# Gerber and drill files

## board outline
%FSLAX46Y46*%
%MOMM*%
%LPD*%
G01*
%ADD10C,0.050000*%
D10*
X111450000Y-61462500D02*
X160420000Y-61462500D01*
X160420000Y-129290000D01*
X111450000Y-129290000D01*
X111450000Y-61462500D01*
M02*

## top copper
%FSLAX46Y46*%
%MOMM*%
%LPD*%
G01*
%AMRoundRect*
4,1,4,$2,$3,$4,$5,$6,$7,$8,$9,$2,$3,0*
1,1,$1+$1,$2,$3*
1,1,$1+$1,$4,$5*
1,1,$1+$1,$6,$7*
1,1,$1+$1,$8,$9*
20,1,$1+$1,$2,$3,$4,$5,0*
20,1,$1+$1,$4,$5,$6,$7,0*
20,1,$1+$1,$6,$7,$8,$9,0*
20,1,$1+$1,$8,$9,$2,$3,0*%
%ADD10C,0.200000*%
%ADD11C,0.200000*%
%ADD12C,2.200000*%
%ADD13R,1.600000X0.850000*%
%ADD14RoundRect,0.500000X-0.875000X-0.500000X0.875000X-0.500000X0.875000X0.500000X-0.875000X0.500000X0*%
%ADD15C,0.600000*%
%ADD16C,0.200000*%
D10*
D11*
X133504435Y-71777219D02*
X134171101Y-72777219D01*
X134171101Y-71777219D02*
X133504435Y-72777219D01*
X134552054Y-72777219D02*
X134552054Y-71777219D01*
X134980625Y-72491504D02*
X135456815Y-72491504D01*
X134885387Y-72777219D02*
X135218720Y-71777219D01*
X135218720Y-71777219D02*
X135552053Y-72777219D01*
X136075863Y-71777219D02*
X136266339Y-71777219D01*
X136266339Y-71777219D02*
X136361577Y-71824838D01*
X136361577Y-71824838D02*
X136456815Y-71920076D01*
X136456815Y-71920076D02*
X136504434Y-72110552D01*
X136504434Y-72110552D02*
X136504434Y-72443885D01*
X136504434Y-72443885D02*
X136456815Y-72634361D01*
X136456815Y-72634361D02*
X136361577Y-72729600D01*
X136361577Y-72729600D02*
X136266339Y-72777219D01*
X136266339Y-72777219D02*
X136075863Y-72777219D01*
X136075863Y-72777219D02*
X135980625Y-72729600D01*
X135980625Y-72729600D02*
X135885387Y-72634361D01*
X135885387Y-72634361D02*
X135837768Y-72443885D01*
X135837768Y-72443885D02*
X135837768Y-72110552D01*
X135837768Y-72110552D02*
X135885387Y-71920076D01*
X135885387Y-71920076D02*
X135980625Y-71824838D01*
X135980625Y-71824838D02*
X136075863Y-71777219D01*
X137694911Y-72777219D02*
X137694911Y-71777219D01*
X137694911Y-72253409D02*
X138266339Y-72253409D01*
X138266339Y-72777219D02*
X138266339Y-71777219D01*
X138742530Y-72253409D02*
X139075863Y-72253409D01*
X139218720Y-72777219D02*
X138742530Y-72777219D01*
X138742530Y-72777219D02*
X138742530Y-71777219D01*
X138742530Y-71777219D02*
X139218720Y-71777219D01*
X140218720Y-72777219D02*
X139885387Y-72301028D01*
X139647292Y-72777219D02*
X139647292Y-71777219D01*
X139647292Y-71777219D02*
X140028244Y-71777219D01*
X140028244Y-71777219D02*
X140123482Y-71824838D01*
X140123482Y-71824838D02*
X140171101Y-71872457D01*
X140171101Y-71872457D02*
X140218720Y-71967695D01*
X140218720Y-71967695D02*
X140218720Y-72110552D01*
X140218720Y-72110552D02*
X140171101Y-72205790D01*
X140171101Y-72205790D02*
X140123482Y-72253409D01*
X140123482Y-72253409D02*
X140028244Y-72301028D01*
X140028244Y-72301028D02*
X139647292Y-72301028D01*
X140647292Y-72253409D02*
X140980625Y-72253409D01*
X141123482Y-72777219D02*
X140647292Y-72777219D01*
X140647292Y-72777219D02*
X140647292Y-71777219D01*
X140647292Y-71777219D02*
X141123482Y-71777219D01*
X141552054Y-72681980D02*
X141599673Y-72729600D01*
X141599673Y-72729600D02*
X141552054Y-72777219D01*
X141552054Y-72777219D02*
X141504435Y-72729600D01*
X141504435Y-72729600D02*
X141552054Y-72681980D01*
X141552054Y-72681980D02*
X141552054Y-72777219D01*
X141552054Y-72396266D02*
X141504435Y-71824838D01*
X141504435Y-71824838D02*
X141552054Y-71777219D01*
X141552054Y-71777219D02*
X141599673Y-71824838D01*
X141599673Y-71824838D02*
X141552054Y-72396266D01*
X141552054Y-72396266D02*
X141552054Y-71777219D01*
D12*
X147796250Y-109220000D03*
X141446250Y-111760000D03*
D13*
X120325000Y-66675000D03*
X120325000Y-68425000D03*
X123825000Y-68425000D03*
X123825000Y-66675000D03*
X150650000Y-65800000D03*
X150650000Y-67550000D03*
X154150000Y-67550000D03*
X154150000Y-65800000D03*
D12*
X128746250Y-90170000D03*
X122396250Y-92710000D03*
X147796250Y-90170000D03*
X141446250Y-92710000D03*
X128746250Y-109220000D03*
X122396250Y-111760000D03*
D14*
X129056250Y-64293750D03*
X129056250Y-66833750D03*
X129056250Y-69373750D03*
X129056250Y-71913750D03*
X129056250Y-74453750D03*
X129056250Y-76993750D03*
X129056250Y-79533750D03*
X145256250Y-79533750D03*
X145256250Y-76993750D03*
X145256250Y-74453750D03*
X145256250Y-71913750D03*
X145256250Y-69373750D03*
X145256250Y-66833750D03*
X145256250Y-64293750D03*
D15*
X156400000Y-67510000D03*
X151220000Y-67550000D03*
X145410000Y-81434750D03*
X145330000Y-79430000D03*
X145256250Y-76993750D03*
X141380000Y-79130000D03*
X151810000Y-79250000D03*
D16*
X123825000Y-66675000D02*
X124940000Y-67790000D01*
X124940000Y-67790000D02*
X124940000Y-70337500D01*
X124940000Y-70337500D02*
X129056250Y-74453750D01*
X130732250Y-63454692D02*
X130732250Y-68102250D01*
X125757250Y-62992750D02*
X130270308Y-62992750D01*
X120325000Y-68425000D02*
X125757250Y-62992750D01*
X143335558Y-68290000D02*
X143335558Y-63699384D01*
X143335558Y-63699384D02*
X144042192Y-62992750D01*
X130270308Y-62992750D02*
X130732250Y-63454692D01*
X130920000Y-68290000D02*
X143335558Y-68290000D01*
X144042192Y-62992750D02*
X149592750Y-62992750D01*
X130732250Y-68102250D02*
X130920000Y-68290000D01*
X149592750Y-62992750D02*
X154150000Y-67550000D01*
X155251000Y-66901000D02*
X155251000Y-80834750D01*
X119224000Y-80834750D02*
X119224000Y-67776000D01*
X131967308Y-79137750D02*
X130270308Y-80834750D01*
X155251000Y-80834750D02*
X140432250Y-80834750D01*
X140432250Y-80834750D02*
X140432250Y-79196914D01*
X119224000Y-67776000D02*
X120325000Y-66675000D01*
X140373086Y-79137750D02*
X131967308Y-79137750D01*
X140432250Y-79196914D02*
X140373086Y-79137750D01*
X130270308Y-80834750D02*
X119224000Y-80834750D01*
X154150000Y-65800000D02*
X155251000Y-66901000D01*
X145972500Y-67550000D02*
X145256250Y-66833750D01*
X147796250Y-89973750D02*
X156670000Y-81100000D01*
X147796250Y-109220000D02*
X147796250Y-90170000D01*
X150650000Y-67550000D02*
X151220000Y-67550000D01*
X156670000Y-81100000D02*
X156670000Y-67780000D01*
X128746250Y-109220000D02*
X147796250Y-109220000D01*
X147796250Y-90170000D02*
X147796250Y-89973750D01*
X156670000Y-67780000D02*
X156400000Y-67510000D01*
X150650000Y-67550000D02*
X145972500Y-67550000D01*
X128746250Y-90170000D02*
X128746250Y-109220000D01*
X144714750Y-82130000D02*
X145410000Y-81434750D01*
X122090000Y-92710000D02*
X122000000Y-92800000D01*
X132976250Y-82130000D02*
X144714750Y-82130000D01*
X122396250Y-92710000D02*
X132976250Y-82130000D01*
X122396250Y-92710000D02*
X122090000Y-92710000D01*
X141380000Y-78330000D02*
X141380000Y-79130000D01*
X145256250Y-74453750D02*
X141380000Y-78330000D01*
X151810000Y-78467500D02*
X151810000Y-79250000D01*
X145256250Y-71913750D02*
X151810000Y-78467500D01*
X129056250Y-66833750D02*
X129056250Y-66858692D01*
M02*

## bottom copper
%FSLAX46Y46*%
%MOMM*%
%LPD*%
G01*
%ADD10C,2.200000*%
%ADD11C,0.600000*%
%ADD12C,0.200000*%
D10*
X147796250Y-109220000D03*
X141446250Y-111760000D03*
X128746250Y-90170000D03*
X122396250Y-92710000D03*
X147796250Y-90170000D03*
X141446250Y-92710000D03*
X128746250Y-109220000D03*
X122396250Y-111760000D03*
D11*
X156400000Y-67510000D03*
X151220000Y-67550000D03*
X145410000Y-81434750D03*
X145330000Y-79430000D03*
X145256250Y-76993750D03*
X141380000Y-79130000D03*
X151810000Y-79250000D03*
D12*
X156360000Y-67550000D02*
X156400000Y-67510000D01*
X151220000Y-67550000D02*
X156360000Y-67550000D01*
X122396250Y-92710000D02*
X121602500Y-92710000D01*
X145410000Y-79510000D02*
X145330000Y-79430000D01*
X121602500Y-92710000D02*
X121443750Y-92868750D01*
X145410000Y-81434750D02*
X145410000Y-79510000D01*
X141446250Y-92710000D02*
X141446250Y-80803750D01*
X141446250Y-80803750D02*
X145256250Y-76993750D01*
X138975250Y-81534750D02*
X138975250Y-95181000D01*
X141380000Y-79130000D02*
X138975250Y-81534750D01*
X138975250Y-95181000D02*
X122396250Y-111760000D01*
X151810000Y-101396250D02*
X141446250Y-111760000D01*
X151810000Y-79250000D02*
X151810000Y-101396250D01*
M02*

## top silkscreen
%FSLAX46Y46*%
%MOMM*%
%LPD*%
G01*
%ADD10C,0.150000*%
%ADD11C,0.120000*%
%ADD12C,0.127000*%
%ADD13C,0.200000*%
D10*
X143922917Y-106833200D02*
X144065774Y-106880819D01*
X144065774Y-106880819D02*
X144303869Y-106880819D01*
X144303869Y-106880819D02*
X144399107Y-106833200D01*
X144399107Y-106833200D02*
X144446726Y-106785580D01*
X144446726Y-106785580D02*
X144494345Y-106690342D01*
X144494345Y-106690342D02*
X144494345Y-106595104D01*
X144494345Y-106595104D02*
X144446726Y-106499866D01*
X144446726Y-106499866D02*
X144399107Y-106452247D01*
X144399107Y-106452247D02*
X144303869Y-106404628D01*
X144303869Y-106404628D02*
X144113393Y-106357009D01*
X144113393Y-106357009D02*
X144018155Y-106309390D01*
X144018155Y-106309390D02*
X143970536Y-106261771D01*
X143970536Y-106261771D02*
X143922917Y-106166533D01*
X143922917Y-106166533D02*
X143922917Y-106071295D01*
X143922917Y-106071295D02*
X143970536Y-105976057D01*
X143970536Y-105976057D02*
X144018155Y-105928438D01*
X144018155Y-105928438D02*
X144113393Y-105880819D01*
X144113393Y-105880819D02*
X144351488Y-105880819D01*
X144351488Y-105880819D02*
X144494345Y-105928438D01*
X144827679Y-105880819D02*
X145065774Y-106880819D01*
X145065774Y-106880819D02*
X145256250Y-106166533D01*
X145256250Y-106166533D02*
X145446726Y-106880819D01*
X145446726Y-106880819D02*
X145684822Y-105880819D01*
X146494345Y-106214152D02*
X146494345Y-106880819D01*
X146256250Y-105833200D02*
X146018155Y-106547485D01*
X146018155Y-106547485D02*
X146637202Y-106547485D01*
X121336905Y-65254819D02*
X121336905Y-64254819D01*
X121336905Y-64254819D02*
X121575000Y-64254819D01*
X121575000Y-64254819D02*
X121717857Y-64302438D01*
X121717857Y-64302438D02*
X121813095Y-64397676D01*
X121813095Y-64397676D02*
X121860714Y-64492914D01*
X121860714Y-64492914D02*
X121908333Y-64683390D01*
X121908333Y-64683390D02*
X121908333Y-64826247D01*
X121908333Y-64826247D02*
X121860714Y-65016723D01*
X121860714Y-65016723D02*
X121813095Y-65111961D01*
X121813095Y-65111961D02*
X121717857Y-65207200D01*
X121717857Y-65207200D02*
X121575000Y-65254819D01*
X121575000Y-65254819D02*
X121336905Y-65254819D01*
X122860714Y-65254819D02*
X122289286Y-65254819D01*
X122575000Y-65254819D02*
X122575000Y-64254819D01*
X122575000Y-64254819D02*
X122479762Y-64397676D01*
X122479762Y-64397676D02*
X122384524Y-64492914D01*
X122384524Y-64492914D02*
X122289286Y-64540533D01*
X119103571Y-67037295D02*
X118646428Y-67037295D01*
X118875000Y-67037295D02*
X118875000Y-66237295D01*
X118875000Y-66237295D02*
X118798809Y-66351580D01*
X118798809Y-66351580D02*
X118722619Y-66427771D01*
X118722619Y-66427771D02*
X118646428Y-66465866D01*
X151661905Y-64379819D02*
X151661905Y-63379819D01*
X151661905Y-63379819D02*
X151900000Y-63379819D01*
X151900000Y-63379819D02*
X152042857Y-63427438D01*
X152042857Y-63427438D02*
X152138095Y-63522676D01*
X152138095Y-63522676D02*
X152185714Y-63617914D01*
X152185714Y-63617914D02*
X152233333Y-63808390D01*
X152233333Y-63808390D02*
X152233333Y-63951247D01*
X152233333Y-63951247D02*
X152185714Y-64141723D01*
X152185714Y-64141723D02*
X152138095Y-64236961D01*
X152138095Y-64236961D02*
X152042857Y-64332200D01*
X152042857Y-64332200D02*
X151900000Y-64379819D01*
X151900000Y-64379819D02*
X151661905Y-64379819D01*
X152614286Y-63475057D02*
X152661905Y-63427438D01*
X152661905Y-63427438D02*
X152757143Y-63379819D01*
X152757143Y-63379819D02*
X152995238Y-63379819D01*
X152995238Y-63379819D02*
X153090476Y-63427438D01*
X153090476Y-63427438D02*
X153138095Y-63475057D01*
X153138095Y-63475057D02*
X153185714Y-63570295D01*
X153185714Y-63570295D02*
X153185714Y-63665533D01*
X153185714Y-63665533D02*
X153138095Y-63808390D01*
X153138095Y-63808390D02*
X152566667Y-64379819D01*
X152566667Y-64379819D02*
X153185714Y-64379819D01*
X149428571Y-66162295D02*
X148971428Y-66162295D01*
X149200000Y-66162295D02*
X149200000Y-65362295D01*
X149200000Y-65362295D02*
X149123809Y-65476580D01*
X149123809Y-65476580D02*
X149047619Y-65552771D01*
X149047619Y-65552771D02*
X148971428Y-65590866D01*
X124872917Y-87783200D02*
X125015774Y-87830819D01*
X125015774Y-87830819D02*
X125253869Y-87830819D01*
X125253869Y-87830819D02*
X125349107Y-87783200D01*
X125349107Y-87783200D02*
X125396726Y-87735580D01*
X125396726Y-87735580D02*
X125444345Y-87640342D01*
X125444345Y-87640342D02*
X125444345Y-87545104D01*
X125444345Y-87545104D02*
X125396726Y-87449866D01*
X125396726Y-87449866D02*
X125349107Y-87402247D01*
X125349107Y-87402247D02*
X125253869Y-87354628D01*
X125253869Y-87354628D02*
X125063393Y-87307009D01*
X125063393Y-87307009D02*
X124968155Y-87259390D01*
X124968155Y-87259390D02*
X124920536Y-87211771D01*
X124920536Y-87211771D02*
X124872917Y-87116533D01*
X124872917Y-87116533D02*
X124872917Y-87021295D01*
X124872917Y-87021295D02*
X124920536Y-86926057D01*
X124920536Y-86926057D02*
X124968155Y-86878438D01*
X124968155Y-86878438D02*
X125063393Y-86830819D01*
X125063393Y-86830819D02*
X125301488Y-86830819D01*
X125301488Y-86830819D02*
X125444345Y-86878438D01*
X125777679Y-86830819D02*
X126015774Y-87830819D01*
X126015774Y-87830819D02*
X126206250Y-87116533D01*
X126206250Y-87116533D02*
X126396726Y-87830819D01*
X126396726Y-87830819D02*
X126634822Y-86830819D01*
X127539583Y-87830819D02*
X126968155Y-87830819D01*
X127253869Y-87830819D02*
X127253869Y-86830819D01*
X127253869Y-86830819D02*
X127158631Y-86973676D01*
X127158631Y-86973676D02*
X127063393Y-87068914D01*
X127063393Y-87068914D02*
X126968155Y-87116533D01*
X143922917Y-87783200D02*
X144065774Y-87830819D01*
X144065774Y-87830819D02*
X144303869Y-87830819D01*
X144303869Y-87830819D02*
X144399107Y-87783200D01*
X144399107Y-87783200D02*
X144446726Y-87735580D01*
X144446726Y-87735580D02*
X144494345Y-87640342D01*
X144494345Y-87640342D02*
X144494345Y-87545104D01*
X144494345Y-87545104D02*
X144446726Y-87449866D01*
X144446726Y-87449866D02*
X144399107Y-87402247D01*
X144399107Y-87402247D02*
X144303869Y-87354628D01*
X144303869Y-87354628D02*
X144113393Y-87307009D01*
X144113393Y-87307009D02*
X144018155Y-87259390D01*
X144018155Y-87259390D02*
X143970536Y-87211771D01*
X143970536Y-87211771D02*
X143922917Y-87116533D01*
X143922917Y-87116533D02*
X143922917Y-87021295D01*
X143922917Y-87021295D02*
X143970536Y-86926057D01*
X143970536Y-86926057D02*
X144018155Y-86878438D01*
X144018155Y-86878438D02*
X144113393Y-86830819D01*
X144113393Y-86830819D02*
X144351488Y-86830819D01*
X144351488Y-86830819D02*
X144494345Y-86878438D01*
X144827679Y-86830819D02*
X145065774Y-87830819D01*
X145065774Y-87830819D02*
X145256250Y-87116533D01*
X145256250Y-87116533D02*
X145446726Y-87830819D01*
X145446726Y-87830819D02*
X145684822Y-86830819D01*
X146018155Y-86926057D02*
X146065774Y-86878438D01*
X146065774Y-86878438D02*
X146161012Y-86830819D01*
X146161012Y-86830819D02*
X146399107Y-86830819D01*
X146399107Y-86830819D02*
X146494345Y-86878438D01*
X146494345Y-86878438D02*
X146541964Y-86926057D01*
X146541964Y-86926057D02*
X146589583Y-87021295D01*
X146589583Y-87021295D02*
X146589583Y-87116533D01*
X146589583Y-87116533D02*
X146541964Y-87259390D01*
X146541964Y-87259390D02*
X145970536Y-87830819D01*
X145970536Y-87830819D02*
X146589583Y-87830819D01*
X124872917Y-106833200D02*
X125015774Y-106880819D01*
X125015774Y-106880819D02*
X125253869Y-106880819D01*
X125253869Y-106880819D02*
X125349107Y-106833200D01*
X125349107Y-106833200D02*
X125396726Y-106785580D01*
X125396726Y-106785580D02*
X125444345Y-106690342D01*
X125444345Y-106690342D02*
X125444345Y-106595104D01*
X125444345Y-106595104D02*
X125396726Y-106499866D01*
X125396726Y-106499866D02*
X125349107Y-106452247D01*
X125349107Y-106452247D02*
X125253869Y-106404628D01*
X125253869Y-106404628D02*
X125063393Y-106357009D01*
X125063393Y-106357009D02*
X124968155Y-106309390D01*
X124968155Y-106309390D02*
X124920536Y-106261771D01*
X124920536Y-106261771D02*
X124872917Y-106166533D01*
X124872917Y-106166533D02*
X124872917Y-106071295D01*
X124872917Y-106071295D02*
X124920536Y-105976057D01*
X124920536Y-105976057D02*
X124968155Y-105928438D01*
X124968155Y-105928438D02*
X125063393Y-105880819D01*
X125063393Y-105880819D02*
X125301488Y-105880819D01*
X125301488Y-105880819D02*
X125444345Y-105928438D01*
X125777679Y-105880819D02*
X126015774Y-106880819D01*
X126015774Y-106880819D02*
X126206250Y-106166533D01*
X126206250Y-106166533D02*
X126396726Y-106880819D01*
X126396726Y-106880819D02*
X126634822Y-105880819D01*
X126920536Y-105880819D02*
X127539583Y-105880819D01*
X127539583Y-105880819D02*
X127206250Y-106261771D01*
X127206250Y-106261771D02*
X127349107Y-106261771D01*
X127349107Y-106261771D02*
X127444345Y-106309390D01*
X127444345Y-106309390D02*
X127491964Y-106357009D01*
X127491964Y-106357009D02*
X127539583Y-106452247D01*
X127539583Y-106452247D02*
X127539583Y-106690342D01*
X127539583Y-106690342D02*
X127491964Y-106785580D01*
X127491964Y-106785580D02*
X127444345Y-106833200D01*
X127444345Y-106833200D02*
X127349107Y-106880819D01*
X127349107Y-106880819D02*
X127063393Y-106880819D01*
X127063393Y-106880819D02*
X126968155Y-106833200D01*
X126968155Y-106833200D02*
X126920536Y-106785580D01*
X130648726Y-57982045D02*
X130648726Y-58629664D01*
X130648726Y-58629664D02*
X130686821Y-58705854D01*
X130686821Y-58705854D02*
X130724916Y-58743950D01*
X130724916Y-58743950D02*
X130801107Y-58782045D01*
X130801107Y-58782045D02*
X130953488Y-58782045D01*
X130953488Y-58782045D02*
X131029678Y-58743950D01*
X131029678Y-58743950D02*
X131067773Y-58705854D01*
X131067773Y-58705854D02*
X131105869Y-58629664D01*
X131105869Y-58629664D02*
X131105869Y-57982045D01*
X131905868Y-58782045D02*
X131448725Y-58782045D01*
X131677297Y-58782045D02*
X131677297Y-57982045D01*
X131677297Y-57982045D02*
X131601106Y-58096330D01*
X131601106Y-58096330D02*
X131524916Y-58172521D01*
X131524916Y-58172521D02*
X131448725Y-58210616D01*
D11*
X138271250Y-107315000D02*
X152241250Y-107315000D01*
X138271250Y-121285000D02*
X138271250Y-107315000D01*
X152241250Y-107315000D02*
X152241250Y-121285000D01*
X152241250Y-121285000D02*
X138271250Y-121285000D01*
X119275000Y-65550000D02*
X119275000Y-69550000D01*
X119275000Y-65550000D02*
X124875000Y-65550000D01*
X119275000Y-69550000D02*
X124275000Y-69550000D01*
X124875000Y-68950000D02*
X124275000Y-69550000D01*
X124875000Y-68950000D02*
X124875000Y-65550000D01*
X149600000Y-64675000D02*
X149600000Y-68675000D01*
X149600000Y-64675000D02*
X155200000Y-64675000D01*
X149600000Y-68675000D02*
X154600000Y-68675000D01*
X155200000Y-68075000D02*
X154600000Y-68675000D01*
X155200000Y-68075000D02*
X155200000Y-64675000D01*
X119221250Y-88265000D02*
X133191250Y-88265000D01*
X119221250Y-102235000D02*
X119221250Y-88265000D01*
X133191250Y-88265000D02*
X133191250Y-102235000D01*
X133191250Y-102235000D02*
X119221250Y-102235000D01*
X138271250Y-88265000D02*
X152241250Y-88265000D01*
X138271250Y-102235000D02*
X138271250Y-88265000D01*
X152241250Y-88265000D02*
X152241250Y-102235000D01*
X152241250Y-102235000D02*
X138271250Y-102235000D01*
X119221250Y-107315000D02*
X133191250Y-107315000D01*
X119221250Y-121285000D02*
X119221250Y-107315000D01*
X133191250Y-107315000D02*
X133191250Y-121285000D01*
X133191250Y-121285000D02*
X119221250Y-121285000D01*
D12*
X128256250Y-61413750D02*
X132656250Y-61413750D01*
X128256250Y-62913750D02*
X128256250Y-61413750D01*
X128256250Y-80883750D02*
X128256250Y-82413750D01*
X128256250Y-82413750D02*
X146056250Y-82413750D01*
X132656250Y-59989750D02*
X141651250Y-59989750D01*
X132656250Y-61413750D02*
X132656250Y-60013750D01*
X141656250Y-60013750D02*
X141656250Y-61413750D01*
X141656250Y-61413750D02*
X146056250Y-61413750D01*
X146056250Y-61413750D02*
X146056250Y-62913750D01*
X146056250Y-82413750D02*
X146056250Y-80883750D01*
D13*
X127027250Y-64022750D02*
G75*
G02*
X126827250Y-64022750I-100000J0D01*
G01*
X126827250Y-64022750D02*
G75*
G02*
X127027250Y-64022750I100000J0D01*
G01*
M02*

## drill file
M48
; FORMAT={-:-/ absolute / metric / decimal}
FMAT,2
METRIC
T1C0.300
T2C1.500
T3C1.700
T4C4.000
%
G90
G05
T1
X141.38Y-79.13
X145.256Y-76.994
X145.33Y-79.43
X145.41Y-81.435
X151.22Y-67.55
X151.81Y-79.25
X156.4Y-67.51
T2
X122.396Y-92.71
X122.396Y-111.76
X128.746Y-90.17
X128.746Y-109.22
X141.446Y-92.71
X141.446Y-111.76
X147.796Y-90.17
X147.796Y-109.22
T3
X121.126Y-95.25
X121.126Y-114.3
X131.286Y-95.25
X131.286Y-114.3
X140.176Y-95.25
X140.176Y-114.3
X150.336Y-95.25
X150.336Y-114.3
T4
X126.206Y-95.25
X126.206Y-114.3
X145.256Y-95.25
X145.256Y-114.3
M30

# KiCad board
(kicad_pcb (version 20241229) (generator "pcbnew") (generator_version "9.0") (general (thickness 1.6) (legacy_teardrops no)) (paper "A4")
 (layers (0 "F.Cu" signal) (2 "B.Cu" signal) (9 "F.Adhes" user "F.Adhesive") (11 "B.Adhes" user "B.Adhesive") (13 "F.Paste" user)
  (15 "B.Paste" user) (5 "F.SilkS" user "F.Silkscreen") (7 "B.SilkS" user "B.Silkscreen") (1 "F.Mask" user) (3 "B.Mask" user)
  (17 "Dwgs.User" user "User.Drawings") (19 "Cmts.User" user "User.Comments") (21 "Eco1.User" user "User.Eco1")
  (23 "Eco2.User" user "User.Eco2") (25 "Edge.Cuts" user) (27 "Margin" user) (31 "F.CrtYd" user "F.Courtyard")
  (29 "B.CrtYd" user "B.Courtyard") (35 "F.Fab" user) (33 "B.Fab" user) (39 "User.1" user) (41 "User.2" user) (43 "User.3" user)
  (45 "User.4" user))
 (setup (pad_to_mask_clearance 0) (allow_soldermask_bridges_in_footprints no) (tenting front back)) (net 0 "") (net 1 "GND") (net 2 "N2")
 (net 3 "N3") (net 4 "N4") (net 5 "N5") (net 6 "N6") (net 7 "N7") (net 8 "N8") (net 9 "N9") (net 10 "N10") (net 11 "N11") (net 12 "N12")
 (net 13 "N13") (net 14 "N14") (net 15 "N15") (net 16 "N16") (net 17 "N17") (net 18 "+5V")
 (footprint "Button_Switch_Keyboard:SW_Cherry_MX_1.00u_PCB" (layer "F.Cu") (at 147.79625 109.22)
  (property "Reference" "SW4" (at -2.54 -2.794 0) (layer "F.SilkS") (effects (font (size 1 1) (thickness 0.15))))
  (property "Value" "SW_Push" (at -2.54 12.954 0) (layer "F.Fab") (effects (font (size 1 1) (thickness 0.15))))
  (fp_line (start -9.525 -1.905) (end 4.445 -1.905) (stroke (width 0.12) (type solid)) (layer "F.SilkS"))
  (fp_line (start -9.525 12.065) (end -9.525 -1.905) (stroke (width 0.12) (type solid)) (layer "F.SilkS"))
  (fp_line (start 4.445 -1.905) (end 4.445 12.065) (stroke (width 0.12) (type solid)) (layer "F.SilkS"))
  (fp_line (start 4.445 12.065) (end -9.525 12.065) (stroke (width 0.12) (type solid)) (layer "F.SilkS"))
  (pad "" np_thru_hole circle (at -7.62 5.08) (size 1.7 1.7) (drill 1.7) (layers "*.Cu" "*.Mask"))
  (pad "" np_thru_hole circle (at -2.54 5.08) (size 4 4) (drill 4) (layers "*.Cu" "*.Mask"))
  (pad "" np_thru_hole circle (at 2.54 5.08) (size 1.7 1.7) (drill 1.7) (layers "*.Cu" "*.Mask"))
  (pad "1" thru_hole circle (at 0 0) (size 2.2 2.2) (drill 1.5) (layers "*.Cu" "*.Mask") (remove_unused_layers no) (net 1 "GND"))
  (pad "2" thru_hole circle (at -6.35 2.54) (size 2.2 2.2) (drill 1.5) (layers "*.Cu" "*.Mask") (remove_unused_layers no) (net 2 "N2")))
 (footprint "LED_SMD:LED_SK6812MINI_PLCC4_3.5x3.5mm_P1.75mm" (layer "F.Cu") (at 122.075 67.55)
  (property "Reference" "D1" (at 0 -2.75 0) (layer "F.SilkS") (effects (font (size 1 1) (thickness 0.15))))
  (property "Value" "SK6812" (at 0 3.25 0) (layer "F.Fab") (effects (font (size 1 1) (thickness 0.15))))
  (fp_line (start -2.8 -2) (end -2.8 2) (stroke (width 0.12) (type default)) (layer "F.SilkS"))
  (fp_line (start -2.8 -2) (end 2.8 -2) (stroke (width 0.12) (type solid)) (layer "F.SilkS"))
  (fp_line (start -2.8 2) (end 2.2 2) (stroke (width 0.12) (type solid)) (layer "F.SilkS"))
  (fp_line (start 2.8 1.4) (end 2.2 2) (stroke (width 0.12) (type default)) (layer "F.SilkS"))
  (fp_line (start 2.8 1.4) (end 2.8 -2) (stroke (width 0.12) (type solid)) (layer "F.SilkS"))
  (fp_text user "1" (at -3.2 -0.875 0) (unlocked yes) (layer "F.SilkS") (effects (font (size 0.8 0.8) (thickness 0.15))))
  (pad "1" smd rect (at -1.75 -0.875) (size 1.6 0.85) (layers "F.Cu" "F.Mask" "F.Paste") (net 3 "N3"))
  (pad "2" smd rect (at -1.75 0.875) (size 1.6 0.85) (layers "F.Cu" "F.Mask" "F.Paste") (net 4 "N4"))
  (pad "3" smd rect (at 1.75 0.875) (size 1.6 0.85) (layers "F.Cu" "F.Mask" "F.Paste") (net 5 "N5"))
  (pad "4" smd rect (at 1.75 -0.875) (size 1.6 0.85) (layers "F.Cu" "F.Mask" "F.Paste") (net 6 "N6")))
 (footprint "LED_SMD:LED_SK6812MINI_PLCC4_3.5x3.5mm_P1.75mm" (layer "F.Cu") (at 152.4 66.675)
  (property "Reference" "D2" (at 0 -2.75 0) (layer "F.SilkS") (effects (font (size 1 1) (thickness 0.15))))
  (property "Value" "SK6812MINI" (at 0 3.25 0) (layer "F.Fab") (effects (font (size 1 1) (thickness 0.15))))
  (fp_line (start -2.8 -2) (end -2.8 2) (stroke (width 0.12) (type default)) (layer "F.SilkS"))
  (fp_line (start -2.8 -2) (end 2.8 -2) (stroke (width 0.12) (type solid)) (layer "F.SilkS"))
  (fp_line (start -2.8 2) (end 2.2 2) (stroke (width 0.12) (type solid)) (layer "F.SilkS"))
  (fp_line (start 2.8 1.4) (end 2.2 2) (stroke (width 0.12) (type default)) (layer "F.SilkS"))
  (fp_line (start 2.8 1.4) (end 2.8 -2) (stroke (width 0.12) (type solid)) (layer "F.SilkS"))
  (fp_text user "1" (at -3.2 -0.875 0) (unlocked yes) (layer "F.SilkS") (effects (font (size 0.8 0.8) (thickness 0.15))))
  (pad "1" smd rect (at -1.75 -0.875) (size 1.6 0.85) (layers "F.Cu" "F.Mask" "F.Paste") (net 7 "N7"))
  (pad "2" smd rect (at -1.75 0.875) (size 1.6 0.85) (layers "F.Cu" "F.Mask" "F.Paste") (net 1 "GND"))
  (pad "3" smd rect (at 1.75 0.875) (size 1.6 0.85) (layers "F.Cu" "F.Mask" "F.Paste") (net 4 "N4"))
  (pad "4" smd rect (at 1.75 -0.875) (size 1.6 0.85) (layers "F.Cu" "F.Mask" "F.Paste") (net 3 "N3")))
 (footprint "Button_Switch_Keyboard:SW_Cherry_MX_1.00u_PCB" (layer "F.Cu") (at 128.74625 90.17)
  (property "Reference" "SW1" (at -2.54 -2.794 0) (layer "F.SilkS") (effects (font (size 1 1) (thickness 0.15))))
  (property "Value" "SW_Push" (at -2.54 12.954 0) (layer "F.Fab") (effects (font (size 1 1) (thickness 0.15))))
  (fp_line (start -9.525 -1.905) (end 4.445 -1.905) (stroke (width 0.12) (type solid)) (layer "F.SilkS"))
  (fp_line (start -9.525 12.065) (end -9.525 -1.905) (stroke (width 0.12) (type solid)) (layer "F.SilkS"))
  (fp_line (start 4.445 -1.905) (end 4.445 12.065) (stroke (width 0.12) (type solid)) (layer "F.SilkS"))
  (fp_line (start 4.445 12.065) (end -9.525 12.065) (stroke (width 0.12) (type solid)) (layer "F.SilkS"))
  (pad "" np_thru_hole circle (at -7.62 5.08) (size 1.7 1.7) (drill 1.7) (layers "*.Cu" "*.Mask"))
  (pad "" np_thru_hole circle (at -2.54 5.08) (size 4 4) (drill 4) (layers "*.Cu" "*.Mask"))
  (pad "" np_thru_hole circle (at 2.54 5.08) (size 1.7 1.7) (drill 1.7) (layers "*.Cu" "*.Mask"))
  (pad "1" thru_hole circle (at 0 0) (size 2.2 2.2) (drill 1.5) (layers "*.Cu" "*.Mask") (remove_unused_layers no) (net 1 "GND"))
  (pad "2" thru_hole circle (at -6.35 2.54) (size 2.2 2.2) (drill 1.5) (layers "*.Cu" "*.Mask") (remove_unused_layers no) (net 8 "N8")))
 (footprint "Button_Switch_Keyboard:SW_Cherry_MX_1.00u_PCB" (layer "F.Cu") (at 147.79625 90.17)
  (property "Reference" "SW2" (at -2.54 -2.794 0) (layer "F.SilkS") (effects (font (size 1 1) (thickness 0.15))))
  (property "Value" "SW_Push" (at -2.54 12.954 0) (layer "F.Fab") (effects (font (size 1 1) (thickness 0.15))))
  (fp_line (start -9.525 -1.905) (end 4.445 -1.905) (stroke (width 0.12) (type solid)) (layer "F.SilkS"))
  (fp_line (start -9.525 12.065) (end -9.525 -1.905) (stroke (width 0.12) (type solid)) (layer "F.SilkS"))
  (fp_line (start 4.445 -1.905) (end 4.445 12.065) (stroke (width 0.12) (type solid)) (layer "F.SilkS"))
  (fp_line (start 4.445 12.065) (end -9.525 12.065) (stroke (width 0.12) (type solid)) (layer "F.SilkS"))
  (pad "" np_thru_hole circle (at -7.62 5.08) (size 1.7 1.7) (drill 1.7) (layers "*.Cu" "*.Mask"))
  (pad "" np_thru_hole circle (at -2.54 5.08) (size 4 4) (drill 4) (layers "*.Cu" "*.Mask"))
  (pad "" np_thru_hole circle (at 2.54 5.08) (size 1.7 1.7) (drill 1.7) (layers "*.Cu" "*.Mask"))
  (pad "1" thru_hole circle (at 0 0) (size 2.2 2.2) (drill 1.5) (layers "*.Cu" "*.Mask") (remove_unused_layers no) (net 1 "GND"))
  (pad "2" thru_hole circle (at -6.35 2.54) (size 2.2 2.2) (drill 1.5) (layers "*.Cu" "*.Mask") (remove_unused_layers no) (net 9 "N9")))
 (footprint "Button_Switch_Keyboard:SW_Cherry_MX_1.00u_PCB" (layer "F.Cu") (at 128.74625 109.22)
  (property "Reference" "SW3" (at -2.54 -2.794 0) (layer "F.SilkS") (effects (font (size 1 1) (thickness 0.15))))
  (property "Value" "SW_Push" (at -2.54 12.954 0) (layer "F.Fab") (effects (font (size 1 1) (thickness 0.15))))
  (fp_line (start -9.525 -1.905) (end 4.445 -1.905) (stroke (width 0.12) (type solid)) (layer "F.SilkS"))
  (fp_line (start -9.525 12.065) (end -9.525 -1.905) (stroke (width 0.12) (type solid)) (layer "F.SilkS"))
  (fp_line (start 4.445 -1.905) (end 4.445 12.065) (stroke (width 0.12) (type solid)) (layer "F.SilkS"))
  (fp_line (start 4.445 12.065) (end -9.525 12.065) (stroke (width 0.12) (type solid)) (layer "F.SilkS"))
  (pad "" np_thru_hole circle (at -7.62 5.08) (size 1.7 1.7) (drill 1.7) (layers "*.Cu" "*.Mask"))
  (pad "" np_thru_hole circle (at -2.54 5.08) (size 4 4) (drill 4) (layers "*.Cu" "*.Mask"))
  (pad "" np_thru_hole circle (at 2.54 5.08) (size 1.7 1.7) (drill 1.7) (layers "*.Cu" "*.Mask"))
  (pad "1" thru_hole circle (at 0 0) (size 2.2 2.2) (drill 1.5) (layers "*.Cu" "*.Mask") (remove_unused_layers no) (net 1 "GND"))
  (pad "2" thru_hole circle (at -6.35 2.54) (size 2.2 2.2) (drill 1.5) (layers "*.Cu" "*.Mask") (remove_unused_layers no) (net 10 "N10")))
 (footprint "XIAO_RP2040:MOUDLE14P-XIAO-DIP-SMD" (layer "F.Cu") (at 137.15625 71.91375)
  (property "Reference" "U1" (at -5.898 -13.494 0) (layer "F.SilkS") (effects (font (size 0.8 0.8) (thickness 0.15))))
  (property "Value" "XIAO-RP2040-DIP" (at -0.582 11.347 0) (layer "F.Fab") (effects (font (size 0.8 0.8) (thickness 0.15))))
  (fp_line (start -8.9 -10.5) (end -4.5 -10.5) (stroke (width 0.127) (type solid)) (layer "F.SilkS"))
  (fp_line (start -8.9 -9) (end -8.9 -10.5) (stroke (width 0.127) (type solid)) (layer "F.SilkS"))
  (fp_line (start -8.9 8.97) (end -8.9 10.5) (stroke (width 0.127) (type solid)) (layer "F.SilkS"))
  (fp_line (start -8.9 10.5) (end 8.9 10.5) (stroke (width 0.127) (type solid)) (layer "F.SilkS"))
  (fp_line (start -4.5 -11.924) (end 4.495 -11.924) (stroke (width 0.127) (type solid)) (layer "F.SilkS"))
  (fp_line (start -4.5 -10.5) (end -4.5 -11.9) (stroke (width 0.127) (type solid)) (layer "F.SilkS"))
  (fp_line (start 4.5 -11.9) (end 4.5 -10.5) (stroke (width 0.127) (type solid)) (layer "F.SilkS"))
  (fp_line (start 4.5 -10.5) (end 8.9 -10.5) (stroke (width 0.127) (type solid)) (layer "F.SilkS"))
  (fp_line (start 8.9 -10.5) (end 8.9 -9) (stroke (width 0.127) (type solid)) (layer "F.SilkS"))
  (fp_line (start 8.9 10.5) (end 8.9 8.97) (stroke (width 0.127) (type solid)) (layer "F.SilkS"))
  (fp_circle (center -10.229 -7.891) (end -10.129 -7.891) (stroke (width 0.2) (type solid)) (fill no) (layer "F.SilkS"))
  (pad "1" smd roundrect (at -8.1 -7.62) (size 2.75 2) (layers "F.Cu" "F.Mask" "F.Paste") (roundrect_rratio 0.25) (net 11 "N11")
   (solder_mask_margin 0.102))
  (pad "2" smd roundrect (at -8.1 -5.08) (size 2.75 2) (layers "F.Cu" "F.Mask" "F.Paste") (roundrect_rratio 0.25) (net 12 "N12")
   (solder_mask_margin 0.102))
  (pad "3" smd roundrect (at -8.1 -2.54) (size 2.75 2) (layers "F.Cu" "F.Mask" "F.Paste") (roundrect_rratio 0.25) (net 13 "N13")
   (solder_mask_margin 0.102))
  (pad "4" smd roundrect (at -8.1 0) (size 2.75 2) (layers "F.Cu" "F.Mask" "F.Paste") (roundrect_rratio 0.25) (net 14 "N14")
   (solder_mask_margin 0.102))
  (pad "5" smd roundrect (at -8.1 2.54) (size 2.75 2) (layers "F.Cu" "F.Mask" "F.Paste") (roundrect_rratio 0.25) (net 6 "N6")
   (solder_mask_margin 0.102))
  (pad "6" smd roundrect (at -8.1 5.08) (size 2.75 2) (layers "F.Cu" "F.Mask" "F.Paste") (roundrect_rratio 0.25) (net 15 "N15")
   (solder_mask_margin 0.102))
  (pad "7" smd roundrect (at -8.1 7.62) (size 2.75 2) (layers "F.Cu" "F.Mask" "F.Paste") (roundrect_rratio 0.25) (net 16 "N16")
   (solder_mask_margin 0.102))
  (pad "8" smd roundrect (at 8.1 7.62) (size 2.75 2) (layers "F.Cu" "F.Mask" "F.Paste") (roundrect_rratio 0.25) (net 8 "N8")
   (solder_mask_margin 0.102))
  (pad "9" smd roundrect (at 8.1 5.08) (size 2.75 2) (layers "F.Cu" "F.Mask" "F.Paste") (roundrect_rratio 0.25) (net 9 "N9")
   (solder_mask_margin 0.102))
  (pad "10" smd roundrect (at 8.1 2.54) (size 2.75 2) (layers "F.Cu" "F.Mask" "F.Paste") (roundrect_rratio 0.25) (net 10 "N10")
   (solder_mask_margin 0.102))
  (pad "11" smd roundrect (at 8.1 0) (size 2.75 2) (layers "F.Cu" "F.Mask" "F.Paste") (roundrect_rratio 0.25) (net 2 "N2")
   (solder_mask_margin 0.102))
  (pad "12" smd roundrect (at 8.1 -2.54) (size 2.75 2) (layers "F.Cu" "F.Mask" "F.Paste") (roundrect_rratio 0.25) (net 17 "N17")
   (solder_mask_margin 0.102))
  (pad "13" smd roundrect (at 8.1 -5.08) (size 2.75 2) (layers "F.Cu" "F.Mask" "F.Paste") (roundrect_rratio 0.25) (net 1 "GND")
   (solder_mask_margin 0.102))
  (pad "14" smd roundrect (at 8.1 -7.62) (size 2.75 2) (layers "F.Cu" "F.Mask" "F.Paste") (roundrect_rratio 0.25) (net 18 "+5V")
   (solder_mask_margin 0.102))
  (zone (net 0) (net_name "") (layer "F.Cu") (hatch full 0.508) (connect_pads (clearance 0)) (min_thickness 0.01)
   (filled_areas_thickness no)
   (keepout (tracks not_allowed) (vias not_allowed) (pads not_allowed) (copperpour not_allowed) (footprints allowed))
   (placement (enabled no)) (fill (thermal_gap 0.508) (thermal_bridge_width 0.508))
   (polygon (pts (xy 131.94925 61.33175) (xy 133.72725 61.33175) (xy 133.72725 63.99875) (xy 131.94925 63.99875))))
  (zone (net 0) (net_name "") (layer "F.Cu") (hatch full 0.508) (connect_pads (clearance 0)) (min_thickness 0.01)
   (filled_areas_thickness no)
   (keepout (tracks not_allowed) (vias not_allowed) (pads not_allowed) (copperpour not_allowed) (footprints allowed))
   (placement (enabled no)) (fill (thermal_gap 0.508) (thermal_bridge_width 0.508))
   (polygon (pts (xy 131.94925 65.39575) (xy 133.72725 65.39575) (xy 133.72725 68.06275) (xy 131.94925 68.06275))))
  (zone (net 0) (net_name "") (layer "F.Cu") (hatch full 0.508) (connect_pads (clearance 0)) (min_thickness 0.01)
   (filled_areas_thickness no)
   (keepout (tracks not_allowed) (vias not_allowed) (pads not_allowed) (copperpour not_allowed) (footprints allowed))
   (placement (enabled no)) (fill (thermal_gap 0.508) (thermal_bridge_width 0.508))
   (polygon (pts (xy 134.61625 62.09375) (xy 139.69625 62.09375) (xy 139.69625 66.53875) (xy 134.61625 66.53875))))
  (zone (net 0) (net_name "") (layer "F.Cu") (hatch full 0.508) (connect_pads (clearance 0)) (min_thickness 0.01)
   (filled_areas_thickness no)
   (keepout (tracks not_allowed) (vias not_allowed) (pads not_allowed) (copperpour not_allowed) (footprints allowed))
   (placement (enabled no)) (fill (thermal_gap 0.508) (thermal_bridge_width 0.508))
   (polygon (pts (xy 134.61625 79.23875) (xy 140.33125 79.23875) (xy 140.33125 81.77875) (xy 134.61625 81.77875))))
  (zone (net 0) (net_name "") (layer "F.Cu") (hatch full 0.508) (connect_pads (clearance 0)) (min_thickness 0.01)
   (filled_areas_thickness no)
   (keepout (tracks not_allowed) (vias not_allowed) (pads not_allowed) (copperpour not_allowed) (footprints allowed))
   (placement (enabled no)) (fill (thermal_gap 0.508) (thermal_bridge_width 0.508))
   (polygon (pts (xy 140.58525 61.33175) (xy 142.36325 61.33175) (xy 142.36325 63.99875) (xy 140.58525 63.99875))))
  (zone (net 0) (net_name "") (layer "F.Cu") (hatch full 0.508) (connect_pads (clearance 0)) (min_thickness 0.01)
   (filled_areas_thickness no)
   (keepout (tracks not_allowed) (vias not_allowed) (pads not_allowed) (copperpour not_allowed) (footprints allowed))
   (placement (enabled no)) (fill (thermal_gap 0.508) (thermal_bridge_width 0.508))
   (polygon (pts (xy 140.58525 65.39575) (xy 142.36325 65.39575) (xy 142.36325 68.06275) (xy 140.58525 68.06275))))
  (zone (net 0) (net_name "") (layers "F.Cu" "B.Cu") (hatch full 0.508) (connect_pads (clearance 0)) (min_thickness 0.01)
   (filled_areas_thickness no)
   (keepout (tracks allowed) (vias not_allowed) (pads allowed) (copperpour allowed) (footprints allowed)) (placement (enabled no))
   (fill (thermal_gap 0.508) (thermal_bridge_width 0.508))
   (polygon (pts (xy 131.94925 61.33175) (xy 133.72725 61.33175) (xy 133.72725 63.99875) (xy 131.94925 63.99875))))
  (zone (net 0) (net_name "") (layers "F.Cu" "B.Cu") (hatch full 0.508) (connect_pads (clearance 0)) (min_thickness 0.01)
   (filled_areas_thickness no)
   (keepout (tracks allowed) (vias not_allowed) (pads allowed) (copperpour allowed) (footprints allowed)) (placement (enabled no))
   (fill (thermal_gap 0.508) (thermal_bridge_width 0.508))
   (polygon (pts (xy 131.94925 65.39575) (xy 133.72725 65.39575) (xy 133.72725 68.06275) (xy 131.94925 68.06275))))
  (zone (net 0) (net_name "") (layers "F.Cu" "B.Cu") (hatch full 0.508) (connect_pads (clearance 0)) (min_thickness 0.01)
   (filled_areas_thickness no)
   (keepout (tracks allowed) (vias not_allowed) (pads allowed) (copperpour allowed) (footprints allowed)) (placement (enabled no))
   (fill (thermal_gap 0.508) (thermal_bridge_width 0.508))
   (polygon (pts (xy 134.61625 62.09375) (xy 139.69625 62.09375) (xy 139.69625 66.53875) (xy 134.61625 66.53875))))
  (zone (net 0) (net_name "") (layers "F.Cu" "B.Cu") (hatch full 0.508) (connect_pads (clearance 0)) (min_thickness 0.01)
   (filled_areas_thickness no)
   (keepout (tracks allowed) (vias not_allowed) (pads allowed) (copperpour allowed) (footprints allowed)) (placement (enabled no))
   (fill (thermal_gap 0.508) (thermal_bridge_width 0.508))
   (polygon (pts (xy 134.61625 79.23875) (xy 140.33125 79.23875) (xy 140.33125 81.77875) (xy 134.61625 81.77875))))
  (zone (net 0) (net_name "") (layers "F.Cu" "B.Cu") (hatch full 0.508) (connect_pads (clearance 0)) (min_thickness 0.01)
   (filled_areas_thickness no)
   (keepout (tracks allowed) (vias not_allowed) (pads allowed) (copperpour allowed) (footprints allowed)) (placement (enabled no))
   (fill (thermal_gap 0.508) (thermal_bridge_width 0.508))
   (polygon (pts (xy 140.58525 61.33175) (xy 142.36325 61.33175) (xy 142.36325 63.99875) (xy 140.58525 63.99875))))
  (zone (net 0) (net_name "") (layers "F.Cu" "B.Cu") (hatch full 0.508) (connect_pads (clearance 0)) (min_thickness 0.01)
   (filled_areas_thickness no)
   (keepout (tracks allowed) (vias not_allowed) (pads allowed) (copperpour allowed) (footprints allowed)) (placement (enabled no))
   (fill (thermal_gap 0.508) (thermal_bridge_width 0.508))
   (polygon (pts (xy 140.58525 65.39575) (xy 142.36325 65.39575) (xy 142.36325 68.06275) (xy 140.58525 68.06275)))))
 (gr_rect (start 111.45 61.4625) (end 160.42 129.29) (stroke (width 0.05) (type default)) (fill no) (layer "Edge.Cuts"))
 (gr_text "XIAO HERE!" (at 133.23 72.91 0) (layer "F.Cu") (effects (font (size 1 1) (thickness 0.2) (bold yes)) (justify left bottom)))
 (segment (start 123.825 66.675) (end 124.94 67.79) (width 0.2) (layer "F.Cu") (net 6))
 (segment (start 124.94 67.79) (end 124.94 70.3375) (width 0.2) (layer "F.Cu") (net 6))
 (segment (start 124.94 70.3375) (end 129.05625 74.45375) (width 0.2) (layer "F.Cu") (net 6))
 (segment (start 130.73225 63.454692) (end 130.73225 68.10225) (width 0.2) (layer "F.Cu") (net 4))
 (segment (start 125.75725 62.99275) (end 130.270308 62.99275) (width 0.2) (layer "F.Cu") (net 4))
 (segment (start 120.325 68.425) (end 125.75725 62.99275) (width 0.2) (layer "F.Cu") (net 4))
 (segment (start 143.335558 68.29) (end 143.335558 63.699384) (width 0.2) (layer "F.Cu") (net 4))
 (segment (start 143.335558 63.699384) (end 144.042192 62.99275) (width 0.2) (layer "F.Cu") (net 4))
 (segment (start 130.270308 62.99275) (end 130.73225 63.454692) (width 0.2) (layer "F.Cu") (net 4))
 (segment (start 130.92 68.29) (end 143.335558 68.29) (width 0.2) (layer "F.Cu") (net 4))
 (segment (start 144.042192 62.99275) (end 149.59275 62.99275) (width 0.2) (layer "F.Cu") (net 4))
 (segment (start 130.73225 68.10225) (end 130.92 68.29) (width 0.2) (layer "F.Cu") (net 4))
 (segment (start 149.59275 62.99275) (end 154.15 67.55) (width 0.2) (layer "F.Cu") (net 4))
 (segment (start 155.251 66.901) (end 155.251 80.83475) (width 0.2) (layer "F.Cu") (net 3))
 (segment (start 119.224 80.83475) (end 119.224 67.776) (width 0.2) (layer "F.Cu") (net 3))
 (segment (start 131.967308 79.13775) (end 130.270308 80.83475) (width 0.2) (layer "F.Cu") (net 3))
 (segment (start 155.251 80.83475) (end 140.43225 80.83475) (width 0.2) (layer "F.Cu") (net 3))
 (segment (start 140.43225 80.83475) (end 140.43225 79.196914) (width 0.2) (layer "F.Cu") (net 3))
 (segment (start 119.224 67.776) (end 120.325 66.675) (width 0.2) (layer "F.Cu") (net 3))
 (segment (start 140.373086 79.13775) (end 131.967308 79.13775) (width 0.2) (layer "F.Cu") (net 3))
 (segment (start 140.43225 79.196914) (end 140.373086 79.13775) (width 0.2) (layer "F.Cu") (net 3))
 (segment (start 130.270308 80.83475) (end 119.224 80.83475) (width 0.2) (layer "F.Cu") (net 3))
 (segment (start 154.15 65.8) (end 155.251 66.901) (width 0.2) (layer "F.Cu") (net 3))
 (segment (start 145.9725 67.55) (end 145.25625 66.83375) (width 0.2) (layer "F.Cu") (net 1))
 (segment (start 147.79625 89.97375) (end 156.67 81.1) (width 0.2) (layer "F.Cu") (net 1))
 (segment (start 147.79625 109.22) (end 147.79625 90.17) (width 0.2) (layer "F.Cu") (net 1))
 (segment (start 150.65 67.55) (end 151.22 67.55) (width 0.2) (layer "F.Cu") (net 1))
 (segment (start 156.67 81.1) (end 156.67 67.78) (width 0.2) (layer "F.Cu") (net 1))
 (segment (start 128.74625 109.22) (end 147.79625 109.22) (width 0.2) (layer "F.Cu") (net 1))
 (segment (start 147.79625 90.17) (end 147.79625 89.97375) (width 0.2) (layer "F.Cu") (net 1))
 (segment (start 156.67 67.78) (end 156.4 67.51) (width 0.2) (layer "F.Cu") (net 1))
 (segment (start 150.65 67.55) (end 145.9725 67.55) (width 0.2) (layer "F.Cu") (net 1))
 (segment (start 128.74625 90.17) (end 128.74625 109.22) (width 0.2) (layer "F.Cu") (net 1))
 (via (at 156.4 67.51) (size 0.6) (drill 0.3) (layers "F.Cu" "B.Cu") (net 1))
 (via (at 151.22 67.55) (size 0.6) (drill 0.3) (layers "F.Cu" "B.Cu") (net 1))
 (segment (start 156.36 67.55) (end 156.4 67.51) (width 0.2) (layer "B.Cu") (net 1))
 (segment (start 151.22 67.55) (end 156.36 67.55) (width 0.2) (layer "B.Cu") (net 1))
 (segment (start 144.71475 82.13) (end 145.41 81.43475) (width 0.2) (layer "F.Cu") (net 8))
 (segment (start 122.09 92.71) (end 122 92.8) (width 0.2) (layer "F.Cu") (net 8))
 (segment (start 132.97625 82.13) (end 144.71475 82.13) (width 0.2) (layer "F.Cu") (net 8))
 (segment (start 122.39625 92.71) (end 132.97625 82.13) (width 0.2) (layer "F.Cu") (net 8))
 (segment (start 122.39625 92.71) (end 122.09 92.71) (width 0.2) (layer "F.Cu") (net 8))
 (via (at 145.41 81.43475) (size 0.6) (drill 0.3) (layers "F.Cu" "B.Cu") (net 8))
 (via (at 145.33 79.43) (size 0.6) (drill 0.3) (layers "F.Cu" "B.Cu") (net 8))
 (segment (start 122.39625 92.71) (end 121.6025 92.71) (width 0.2) (layer "B.Cu") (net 8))
 (segment (start 145.41 79.51) (end 145.33 79.43) (width 0.2) (layer "B.Cu") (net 8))
 (segment (start 121.6025 92.71) (end 121.44375 92.86875) (width 0.2) (layer "B.Cu") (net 8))
 (segment (start 145.41 81.43475) (end 145.41 79.51) (width 0.2) (layer "B.Cu") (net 8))
 (via (at 145.25625 76.99375) (size 0.6) (drill 0.3) (layers "F.Cu" "B.Cu") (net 9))
 (segment (start 141.44625 92.71) (end 141.44625 80.80375) (width 0.2) (layer "B.Cu") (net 9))
 (segment (start 141.44625 80.80375) (end 145.25625 76.99375) (width 0.2) (layer "B.Cu") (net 9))
 (segment (start 141.38 78.33) (end 141.38 79.13) (width 0.2) (layer "F.Cu") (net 10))
 (segment (start 145.25625 74.45375) (end 141.38 78.33) (width 0.2) (layer "F.Cu") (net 10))
 (via (at 141.38 79.13) (size 0.6) (drill 0.3) (layers "F.Cu" "B.Cu") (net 10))
 (segment (start 138.97525 81.53475) (end 138.97525 95.181) (width 0.2) (layer "B.Cu") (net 10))
 (segment (start 141.38 79.13) (end 138.97525 81.53475) (width 0.2) (layer "B.Cu") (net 10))
 (segment (start 138.97525 95.181) (end 122.39625 111.76) (width 0.2) (layer "B.Cu") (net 10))
 (segment (start 151.81 78.4675) (end 151.81 79.25) (width 0.2) (layer "F.Cu") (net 2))
 (segment (start 145.25625 71.91375) (end 151.81 78.4675) (width 0.2) (layer "F.Cu") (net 2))
 (via (at 151.81 79.25) (size 0.6) (drill 0.3) (layers "F.Cu" "B.Cu") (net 2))
 (segment (start 151.81 101.39625) (end 141.44625 111.76) (width 0.2) (layer "B.Cu") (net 2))
 (segment (start 151.81 79.25) (end 151.81 101.39625) (width 0.2) (layer "B.Cu") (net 2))
 (segment (start 129.05625 66.83375) (end 129.05625 66.858692) (width 0.2) (layer "F.Cu") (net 12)))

